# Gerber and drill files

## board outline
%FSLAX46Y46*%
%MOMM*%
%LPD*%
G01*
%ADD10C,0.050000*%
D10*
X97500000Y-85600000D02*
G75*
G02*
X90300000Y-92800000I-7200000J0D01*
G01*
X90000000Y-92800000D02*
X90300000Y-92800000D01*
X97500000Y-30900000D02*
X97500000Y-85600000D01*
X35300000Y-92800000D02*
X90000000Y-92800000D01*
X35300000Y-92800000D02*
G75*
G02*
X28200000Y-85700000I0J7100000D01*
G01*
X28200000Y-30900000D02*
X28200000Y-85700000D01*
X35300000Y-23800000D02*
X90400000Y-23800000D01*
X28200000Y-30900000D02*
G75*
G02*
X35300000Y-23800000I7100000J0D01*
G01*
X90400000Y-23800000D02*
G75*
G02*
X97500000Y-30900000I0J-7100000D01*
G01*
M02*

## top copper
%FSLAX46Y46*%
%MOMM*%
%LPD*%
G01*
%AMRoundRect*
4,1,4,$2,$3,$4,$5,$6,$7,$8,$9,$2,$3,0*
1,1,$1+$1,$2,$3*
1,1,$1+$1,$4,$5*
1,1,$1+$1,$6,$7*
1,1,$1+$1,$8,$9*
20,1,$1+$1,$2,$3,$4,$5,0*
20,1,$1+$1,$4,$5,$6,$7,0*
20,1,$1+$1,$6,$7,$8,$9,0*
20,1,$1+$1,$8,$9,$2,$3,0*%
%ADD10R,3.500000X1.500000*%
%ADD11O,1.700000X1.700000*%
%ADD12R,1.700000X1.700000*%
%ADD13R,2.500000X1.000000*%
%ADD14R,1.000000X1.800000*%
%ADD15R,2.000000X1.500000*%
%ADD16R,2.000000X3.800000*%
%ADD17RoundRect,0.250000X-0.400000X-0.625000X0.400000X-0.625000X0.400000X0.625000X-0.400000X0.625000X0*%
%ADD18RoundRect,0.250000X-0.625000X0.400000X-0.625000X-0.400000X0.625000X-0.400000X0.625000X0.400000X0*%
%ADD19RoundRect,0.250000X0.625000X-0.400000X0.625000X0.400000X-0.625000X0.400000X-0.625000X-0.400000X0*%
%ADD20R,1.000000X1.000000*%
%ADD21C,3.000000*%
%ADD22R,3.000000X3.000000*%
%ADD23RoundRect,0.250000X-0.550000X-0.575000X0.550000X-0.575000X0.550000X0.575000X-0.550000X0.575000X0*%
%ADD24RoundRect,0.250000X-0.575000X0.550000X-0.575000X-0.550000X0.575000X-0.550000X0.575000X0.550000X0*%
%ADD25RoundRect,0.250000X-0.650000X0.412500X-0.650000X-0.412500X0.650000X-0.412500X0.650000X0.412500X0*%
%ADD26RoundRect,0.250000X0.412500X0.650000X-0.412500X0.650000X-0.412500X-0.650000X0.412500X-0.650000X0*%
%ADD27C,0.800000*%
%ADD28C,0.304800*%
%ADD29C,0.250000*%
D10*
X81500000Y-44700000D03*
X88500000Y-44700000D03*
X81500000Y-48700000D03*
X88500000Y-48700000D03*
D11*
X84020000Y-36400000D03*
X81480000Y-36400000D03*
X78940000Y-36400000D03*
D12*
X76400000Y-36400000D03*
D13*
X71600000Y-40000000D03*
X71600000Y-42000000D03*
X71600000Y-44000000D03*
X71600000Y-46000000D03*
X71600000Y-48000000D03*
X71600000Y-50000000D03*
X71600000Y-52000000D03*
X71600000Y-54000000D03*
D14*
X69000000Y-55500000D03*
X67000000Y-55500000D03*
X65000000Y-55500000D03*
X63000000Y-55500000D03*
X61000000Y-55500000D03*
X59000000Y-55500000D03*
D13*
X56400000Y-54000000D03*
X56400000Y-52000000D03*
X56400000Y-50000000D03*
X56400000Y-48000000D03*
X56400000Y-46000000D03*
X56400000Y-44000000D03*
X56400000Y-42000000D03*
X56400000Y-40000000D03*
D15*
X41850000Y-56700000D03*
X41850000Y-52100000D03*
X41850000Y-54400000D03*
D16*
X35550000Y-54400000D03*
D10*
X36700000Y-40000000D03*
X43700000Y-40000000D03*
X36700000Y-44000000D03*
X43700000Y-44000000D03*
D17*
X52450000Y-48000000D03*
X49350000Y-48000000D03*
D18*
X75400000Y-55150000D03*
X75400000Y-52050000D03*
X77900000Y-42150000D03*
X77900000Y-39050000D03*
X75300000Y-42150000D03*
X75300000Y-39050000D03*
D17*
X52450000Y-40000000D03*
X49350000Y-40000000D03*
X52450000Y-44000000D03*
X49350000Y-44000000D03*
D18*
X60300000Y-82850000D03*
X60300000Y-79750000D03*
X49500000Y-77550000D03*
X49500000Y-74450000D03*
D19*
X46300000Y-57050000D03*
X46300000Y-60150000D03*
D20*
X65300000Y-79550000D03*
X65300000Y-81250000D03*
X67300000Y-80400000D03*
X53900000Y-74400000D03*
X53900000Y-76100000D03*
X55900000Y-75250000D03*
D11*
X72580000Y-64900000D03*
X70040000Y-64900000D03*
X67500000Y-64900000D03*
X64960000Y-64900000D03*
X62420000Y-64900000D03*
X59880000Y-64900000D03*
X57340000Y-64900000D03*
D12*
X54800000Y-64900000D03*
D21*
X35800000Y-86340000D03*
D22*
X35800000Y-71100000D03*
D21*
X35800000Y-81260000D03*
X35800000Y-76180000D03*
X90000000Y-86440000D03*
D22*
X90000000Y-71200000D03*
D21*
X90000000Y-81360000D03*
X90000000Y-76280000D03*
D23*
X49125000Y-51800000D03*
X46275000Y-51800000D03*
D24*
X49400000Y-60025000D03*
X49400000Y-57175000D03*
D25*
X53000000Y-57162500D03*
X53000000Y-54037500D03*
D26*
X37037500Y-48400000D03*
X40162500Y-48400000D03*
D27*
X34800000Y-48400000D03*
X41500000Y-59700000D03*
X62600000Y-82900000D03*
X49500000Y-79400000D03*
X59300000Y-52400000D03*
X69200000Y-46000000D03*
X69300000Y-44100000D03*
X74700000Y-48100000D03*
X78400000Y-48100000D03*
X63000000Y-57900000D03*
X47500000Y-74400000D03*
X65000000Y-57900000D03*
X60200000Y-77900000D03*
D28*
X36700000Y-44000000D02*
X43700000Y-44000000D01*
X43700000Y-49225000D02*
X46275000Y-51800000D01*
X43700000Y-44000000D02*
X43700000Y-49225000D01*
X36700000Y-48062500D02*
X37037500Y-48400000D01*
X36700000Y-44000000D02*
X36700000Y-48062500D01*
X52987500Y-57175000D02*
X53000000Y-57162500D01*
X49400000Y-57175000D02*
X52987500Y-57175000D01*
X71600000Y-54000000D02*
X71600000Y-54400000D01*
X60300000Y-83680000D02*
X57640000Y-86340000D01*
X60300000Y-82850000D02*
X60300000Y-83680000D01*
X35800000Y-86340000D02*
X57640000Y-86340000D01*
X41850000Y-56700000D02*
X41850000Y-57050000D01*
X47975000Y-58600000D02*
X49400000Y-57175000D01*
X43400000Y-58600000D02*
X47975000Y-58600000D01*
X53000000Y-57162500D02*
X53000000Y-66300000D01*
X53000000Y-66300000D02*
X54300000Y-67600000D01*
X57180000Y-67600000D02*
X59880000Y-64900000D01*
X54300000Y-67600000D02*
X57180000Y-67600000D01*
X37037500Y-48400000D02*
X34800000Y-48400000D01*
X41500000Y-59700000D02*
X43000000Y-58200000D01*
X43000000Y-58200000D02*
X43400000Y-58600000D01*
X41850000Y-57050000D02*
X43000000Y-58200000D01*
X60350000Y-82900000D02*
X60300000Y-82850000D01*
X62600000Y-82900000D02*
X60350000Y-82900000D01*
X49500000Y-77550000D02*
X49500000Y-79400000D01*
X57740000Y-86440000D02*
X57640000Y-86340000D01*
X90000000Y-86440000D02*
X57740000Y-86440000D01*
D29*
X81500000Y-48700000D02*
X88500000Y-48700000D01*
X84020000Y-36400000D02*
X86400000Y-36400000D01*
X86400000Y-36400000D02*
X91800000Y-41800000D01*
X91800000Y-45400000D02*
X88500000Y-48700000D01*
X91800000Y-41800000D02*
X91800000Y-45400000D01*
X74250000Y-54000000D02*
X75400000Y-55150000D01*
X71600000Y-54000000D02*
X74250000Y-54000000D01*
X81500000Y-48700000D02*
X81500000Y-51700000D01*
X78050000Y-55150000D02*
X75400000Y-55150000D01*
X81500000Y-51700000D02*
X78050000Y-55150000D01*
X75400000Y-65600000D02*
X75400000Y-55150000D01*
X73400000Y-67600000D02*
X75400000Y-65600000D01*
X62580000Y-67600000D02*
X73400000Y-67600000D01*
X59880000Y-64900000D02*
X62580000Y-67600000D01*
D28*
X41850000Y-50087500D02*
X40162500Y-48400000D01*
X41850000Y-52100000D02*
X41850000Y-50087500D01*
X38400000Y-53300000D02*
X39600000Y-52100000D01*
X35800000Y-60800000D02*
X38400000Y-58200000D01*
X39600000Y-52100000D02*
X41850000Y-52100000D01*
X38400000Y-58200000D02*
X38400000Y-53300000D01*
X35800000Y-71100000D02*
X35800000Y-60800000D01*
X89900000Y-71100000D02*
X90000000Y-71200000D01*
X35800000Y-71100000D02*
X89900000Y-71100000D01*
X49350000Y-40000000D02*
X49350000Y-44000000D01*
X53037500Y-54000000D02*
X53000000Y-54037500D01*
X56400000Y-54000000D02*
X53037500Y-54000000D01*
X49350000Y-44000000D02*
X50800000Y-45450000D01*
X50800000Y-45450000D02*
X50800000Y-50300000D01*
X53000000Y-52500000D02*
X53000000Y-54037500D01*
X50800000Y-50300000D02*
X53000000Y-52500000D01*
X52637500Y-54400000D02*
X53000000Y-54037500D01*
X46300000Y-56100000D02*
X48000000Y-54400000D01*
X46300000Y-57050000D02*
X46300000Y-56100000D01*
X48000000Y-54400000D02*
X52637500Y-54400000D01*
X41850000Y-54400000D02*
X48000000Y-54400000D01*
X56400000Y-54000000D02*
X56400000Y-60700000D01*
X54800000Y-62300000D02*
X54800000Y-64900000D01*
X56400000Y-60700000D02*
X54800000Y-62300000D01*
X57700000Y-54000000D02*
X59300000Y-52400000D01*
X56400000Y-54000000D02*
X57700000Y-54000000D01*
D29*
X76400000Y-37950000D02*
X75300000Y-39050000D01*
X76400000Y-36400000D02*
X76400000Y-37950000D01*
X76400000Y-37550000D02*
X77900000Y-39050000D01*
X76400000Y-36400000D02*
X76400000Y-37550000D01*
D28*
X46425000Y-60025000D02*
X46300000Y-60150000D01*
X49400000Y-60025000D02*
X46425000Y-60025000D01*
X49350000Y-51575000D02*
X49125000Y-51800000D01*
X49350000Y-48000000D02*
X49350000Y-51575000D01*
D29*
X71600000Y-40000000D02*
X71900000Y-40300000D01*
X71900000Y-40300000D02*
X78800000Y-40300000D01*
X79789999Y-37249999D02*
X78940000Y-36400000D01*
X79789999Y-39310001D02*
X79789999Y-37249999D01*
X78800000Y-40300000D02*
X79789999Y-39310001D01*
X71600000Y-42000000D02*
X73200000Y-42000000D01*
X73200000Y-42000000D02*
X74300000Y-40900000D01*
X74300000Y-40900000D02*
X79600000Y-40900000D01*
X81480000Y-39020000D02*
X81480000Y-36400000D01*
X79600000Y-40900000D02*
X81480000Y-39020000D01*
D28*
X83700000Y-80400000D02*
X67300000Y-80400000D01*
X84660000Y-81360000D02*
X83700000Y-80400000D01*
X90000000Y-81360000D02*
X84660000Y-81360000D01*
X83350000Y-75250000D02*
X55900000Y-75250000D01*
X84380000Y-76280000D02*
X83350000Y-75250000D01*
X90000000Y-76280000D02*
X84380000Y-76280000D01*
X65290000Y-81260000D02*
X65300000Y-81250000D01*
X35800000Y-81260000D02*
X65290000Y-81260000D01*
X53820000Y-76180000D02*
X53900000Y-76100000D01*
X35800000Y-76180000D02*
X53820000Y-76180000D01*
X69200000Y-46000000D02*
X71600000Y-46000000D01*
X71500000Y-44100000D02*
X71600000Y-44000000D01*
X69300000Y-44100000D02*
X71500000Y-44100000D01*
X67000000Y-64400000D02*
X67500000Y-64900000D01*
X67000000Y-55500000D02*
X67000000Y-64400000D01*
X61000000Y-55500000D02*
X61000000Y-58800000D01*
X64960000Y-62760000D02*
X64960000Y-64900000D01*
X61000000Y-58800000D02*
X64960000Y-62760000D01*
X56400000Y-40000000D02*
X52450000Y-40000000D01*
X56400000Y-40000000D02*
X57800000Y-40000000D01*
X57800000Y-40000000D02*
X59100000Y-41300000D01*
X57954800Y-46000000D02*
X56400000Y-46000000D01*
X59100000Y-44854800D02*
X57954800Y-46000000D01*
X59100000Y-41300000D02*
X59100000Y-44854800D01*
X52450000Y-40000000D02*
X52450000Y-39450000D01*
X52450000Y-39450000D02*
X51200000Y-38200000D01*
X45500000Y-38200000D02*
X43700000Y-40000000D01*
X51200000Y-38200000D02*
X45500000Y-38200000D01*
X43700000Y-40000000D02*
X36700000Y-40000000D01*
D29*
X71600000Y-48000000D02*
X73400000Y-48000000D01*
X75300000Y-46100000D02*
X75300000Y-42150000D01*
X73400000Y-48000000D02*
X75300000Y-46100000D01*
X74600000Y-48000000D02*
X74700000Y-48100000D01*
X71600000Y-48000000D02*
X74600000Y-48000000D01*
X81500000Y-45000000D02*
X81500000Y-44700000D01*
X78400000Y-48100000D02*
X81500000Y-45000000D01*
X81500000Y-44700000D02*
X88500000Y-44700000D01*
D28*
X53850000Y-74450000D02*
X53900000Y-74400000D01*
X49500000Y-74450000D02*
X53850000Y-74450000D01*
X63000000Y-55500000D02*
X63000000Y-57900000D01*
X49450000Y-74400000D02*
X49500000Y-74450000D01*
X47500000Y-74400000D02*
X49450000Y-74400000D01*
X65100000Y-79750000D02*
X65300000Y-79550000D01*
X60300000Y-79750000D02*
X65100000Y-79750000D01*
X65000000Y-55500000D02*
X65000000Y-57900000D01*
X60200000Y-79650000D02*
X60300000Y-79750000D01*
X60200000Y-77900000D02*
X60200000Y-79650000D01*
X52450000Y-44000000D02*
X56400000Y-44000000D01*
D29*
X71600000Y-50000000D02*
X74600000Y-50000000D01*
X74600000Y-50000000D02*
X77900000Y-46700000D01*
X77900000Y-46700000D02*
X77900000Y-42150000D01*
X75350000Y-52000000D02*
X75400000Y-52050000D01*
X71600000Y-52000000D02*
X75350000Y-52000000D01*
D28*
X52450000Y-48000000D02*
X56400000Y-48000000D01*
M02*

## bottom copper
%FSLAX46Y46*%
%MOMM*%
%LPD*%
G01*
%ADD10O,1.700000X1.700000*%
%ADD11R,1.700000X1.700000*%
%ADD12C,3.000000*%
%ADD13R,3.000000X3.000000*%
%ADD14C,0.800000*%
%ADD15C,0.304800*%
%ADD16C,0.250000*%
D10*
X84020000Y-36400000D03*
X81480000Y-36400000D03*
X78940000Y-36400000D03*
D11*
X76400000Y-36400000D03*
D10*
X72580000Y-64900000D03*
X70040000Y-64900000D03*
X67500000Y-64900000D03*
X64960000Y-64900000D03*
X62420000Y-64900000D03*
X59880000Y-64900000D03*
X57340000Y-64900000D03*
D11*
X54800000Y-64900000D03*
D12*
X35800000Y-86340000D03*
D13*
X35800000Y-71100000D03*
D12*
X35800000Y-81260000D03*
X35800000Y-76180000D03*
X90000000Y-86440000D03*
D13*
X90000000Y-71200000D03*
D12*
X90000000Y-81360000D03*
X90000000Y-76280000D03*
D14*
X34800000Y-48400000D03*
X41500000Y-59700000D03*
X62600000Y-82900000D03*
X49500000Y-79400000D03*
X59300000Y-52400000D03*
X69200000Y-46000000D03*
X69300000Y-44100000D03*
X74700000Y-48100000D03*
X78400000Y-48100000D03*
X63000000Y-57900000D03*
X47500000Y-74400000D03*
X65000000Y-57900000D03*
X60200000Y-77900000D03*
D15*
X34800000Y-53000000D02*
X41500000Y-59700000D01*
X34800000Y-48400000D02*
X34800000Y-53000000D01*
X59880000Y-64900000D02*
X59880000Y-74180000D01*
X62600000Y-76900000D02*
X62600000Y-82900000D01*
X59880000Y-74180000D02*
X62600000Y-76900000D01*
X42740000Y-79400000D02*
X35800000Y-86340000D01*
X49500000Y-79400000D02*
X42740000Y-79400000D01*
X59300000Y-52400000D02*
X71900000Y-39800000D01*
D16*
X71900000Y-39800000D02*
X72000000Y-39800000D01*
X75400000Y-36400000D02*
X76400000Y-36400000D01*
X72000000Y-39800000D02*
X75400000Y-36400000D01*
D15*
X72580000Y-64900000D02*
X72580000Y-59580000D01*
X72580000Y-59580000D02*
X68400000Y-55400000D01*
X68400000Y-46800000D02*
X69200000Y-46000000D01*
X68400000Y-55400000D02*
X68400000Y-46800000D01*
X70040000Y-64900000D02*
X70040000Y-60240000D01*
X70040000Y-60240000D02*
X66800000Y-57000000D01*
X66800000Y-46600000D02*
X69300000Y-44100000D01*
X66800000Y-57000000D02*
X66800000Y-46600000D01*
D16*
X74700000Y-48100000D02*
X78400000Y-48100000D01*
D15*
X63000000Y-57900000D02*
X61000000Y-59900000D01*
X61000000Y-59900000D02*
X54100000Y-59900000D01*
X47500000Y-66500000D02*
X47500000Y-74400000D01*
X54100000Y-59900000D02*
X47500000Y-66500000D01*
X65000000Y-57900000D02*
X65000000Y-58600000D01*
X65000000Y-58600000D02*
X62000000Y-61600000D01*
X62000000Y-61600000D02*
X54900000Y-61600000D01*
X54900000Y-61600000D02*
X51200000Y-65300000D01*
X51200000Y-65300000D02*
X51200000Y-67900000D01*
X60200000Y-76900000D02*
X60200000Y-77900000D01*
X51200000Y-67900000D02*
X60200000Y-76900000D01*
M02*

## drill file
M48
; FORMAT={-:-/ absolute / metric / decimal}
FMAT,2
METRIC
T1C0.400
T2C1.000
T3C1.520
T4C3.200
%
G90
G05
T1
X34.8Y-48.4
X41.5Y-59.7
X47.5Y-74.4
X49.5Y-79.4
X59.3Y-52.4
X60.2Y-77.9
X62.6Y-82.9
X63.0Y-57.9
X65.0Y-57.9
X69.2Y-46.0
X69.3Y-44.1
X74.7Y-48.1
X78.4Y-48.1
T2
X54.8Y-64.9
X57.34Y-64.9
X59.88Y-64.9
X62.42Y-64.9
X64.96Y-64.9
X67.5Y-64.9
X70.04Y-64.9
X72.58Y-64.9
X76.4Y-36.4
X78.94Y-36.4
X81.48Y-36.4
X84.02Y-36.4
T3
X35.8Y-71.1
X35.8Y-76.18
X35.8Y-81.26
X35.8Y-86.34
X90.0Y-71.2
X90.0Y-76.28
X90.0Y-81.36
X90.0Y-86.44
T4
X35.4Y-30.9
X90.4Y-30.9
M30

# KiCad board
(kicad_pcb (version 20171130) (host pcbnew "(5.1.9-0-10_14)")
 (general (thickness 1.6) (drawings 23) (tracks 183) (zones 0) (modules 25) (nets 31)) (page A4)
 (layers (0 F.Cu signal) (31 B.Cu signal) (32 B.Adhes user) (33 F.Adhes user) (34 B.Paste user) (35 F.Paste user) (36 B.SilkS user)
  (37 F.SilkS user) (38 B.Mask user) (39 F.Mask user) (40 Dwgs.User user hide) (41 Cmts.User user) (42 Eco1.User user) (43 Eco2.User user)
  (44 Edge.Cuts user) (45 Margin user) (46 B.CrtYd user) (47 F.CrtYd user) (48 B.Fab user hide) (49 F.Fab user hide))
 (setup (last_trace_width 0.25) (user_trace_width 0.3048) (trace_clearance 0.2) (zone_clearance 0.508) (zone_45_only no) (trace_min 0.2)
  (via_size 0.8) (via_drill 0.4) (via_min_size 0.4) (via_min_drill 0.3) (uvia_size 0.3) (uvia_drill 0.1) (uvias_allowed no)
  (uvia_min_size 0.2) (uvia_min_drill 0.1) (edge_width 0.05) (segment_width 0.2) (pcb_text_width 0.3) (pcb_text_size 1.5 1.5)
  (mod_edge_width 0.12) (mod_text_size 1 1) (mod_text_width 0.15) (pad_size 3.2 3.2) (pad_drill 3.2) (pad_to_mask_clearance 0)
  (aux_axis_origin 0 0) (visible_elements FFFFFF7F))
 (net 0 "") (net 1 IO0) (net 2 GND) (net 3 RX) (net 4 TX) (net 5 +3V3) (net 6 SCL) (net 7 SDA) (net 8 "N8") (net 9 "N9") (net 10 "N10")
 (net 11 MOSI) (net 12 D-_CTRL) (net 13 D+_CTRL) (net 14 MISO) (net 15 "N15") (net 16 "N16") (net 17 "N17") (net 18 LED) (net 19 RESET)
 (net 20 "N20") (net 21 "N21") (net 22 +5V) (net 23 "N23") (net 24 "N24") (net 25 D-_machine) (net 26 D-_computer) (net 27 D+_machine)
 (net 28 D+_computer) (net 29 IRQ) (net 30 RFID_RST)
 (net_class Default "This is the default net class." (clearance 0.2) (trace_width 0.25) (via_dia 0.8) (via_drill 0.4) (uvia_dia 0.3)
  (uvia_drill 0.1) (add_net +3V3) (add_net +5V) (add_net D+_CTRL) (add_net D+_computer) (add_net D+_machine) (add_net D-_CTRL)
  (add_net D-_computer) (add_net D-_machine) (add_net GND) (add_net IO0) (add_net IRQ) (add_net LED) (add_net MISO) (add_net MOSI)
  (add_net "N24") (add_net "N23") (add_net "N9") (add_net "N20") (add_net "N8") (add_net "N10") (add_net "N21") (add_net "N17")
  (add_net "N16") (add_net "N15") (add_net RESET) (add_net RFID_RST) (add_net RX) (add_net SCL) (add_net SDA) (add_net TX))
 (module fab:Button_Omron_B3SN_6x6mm (layer F.Cu) (at 85 46.7)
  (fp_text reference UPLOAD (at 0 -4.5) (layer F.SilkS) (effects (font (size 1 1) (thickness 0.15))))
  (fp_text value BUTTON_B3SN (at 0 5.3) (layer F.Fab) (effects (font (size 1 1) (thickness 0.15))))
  (pad 1 smd rect (at -3.5 -2) (size 3.5 1.5) (layers F.Cu F.Paste F.Mask) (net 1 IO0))
  (pad 1 smd rect (at 3.5 -2) (size 3.5 1.5) (layers F.Cu F.Paste F.Mask) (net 1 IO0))
  (pad 2 smd rect (at -3.5 2) (size 3.5 1.5) (layers F.Cu F.Paste F.Mask) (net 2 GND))
  (pad 2 smd rect (at 3.5 2) (size 3.5 1.5) (layers F.Cu F.Paste F.Mask) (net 2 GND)))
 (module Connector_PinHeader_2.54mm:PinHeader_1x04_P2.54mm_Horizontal (layer F.Cu) (at 76.4 36.4 90)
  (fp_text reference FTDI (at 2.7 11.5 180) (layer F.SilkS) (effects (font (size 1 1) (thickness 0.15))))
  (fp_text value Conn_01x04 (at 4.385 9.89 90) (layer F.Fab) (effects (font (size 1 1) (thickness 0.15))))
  (pad 4 thru_hole oval (at 0 7.62 90) (size 1.7 1.7) (drill 1) (layers *.Cu *.Mask) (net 2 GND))
  (pad 3 thru_hole oval (at 0 5.08 90) (size 1.7 1.7) (drill 1) (layers *.Cu *.Mask) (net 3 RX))
  (pad 2 thru_hole oval (at 0 2.54 90) (size 1.7 1.7) (drill 1) (layers *.Cu *.Mask) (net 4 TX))
  (pad 1 thru_hole rect (at 0 0 90) (size 1.7 1.7) (drill 1) (layers *.Cu *.Mask) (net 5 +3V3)))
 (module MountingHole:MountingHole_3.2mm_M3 (layer F.Cu) (at 90.4 30.9)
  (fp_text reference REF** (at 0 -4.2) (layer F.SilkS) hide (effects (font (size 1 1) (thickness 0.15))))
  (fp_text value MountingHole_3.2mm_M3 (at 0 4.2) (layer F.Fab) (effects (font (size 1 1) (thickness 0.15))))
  (pad 1 np_thru_hole circle (at 0 0) (size 3.2 3.2) (drill 3.2) (layers *.Cu *.Mask)))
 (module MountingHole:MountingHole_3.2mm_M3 (layer F.Cu) (at 35.4 30.9)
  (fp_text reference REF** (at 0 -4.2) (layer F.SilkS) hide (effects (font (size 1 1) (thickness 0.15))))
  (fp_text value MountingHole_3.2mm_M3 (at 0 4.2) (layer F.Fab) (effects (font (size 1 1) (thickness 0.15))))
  (pad 1 np_thru_hole circle (at 0 0) (size 3.2 3.2) (drill 3.2) (layers *.Cu *.Mask)))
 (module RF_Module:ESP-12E (layer F.Cu) (at 64 43.5)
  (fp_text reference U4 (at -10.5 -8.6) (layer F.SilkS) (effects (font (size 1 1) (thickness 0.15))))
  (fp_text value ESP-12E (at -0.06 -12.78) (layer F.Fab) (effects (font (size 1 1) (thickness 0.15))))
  (pad 22 smd rect (at 7.6 -3.5) (size 2.5 1) (layers F.Cu F.Paste F.Mask) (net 4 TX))
  (pad 21 smd rect (at 7.6 -1.5) (size 2.5 1) (layers F.Cu F.Paste F.Mask) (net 3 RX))
  (pad 20 smd rect (at 7.6 0.5) (size 2.5 1) (layers F.Cu F.Paste F.Mask) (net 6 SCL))
  (pad 19 smd rect (at 7.6 2.5) (size 2.5 1) (layers F.Cu F.Paste F.Mask) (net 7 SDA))
  (pad 18 smd rect (at 7.6 4.5) (size 2.5 1) (layers F.Cu F.Paste F.Mask) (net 1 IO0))
  (pad 17 smd rect (at 7.6 6.5) (size 2.5 1) (layers F.Cu F.Paste F.Mask) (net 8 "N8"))
  (pad 16 smd rect (at 7.6 8.5) (size 2.5 1) (layers F.Cu F.Paste F.Mask) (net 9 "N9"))
  (pad 15 smd rect (at 7.6 10.5) (size 2.5 1) (layers F.Cu F.Paste F.Mask) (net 2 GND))
  (pad 14 smd rect (at 5 12) (size 1 1.8) (layers F.Cu F.Paste F.Mask) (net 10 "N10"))
  (pad 13 smd rect (at 3 12) (size 1 1.8) (layers F.Cu F.Paste F.Mask) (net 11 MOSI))
  (pad 12 smd rect (at 1 12) (size 1 1.8) (layers F.Cu F.Paste F.Mask) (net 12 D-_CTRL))
  (pad 11 smd rect (at -1 12) (size 1 1.8) (layers F.Cu F.Paste F.Mask) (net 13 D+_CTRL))
  (pad 10 smd rect (at -3 12) (size 1 1.8) (layers F.Cu F.Paste F.Mask) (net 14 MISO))
  (pad 9 smd rect (at -5 12) (size 1 1.8) (layers F.Cu F.Paste F.Mask) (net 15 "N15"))
  (pad 8 smd rect (at -7.6 10.5) (size 2.5 1) (layers F.Cu F.Paste F.Mask) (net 5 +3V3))
  (pad 7 smd rect (at -7.6 8.5) (size 2.5 1) (layers F.Cu F.Paste F.Mask) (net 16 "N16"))
  (pad 6 smd rect (at -7.6 6.5) (size 2.5 1) (layers F.Cu F.Paste F.Mask) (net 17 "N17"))
  (pad 5 smd rect (at -7.6 4.5) (size 2.5 1) (layers F.Cu F.Paste F.Mask) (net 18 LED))
  (pad 4 smd rect (at -7.6 2.5) (size 2.5 1) (layers F.Cu F.Paste F.Mask) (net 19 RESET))
  (pad 3 smd rect (at -7.6 0.5) (size 2.5 1) (layers F.Cu F.Paste F.Mask) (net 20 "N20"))
  (pad 2 smd rect (at -7.6 -1.5) (size 2.5 1) (layers F.Cu F.Paste F.Mask) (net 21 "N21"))
  (pad 1 smd rect (at -7.6 -3.5) (size 2.5 1) (layers F.Cu F.Paste F.Mask) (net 19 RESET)))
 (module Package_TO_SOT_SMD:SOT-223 (layer F.Cu) (at 38.7 54.4 180)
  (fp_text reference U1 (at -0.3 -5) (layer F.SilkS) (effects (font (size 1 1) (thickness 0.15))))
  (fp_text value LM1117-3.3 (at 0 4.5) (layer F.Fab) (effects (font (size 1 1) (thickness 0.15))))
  (pad 1 smd rect (at -3.15 -2.3 180) (size 2 1.5) (layers F.Cu F.Paste F.Mask) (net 2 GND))
  (pad 3 smd rect (at -3.15 2.3 180) (size 2 1.5) (layers F.Cu F.Paste F.Mask) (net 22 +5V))
  (pad 2 smd rect (at -3.15 0 180) (size 2 1.5) (layers F.Cu F.Paste F.Mask) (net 5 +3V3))
  (pad 4 smd rect (at 3.15 0 180) (size 2 3.8) (layers F.Cu F.Paste F.Mask)))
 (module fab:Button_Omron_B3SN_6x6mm (layer F.Cu) (at 40.2 42)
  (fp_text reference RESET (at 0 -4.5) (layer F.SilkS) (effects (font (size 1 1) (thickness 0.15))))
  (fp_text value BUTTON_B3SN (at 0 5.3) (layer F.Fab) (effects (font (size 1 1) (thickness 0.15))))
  (pad 1 smd rect (at -3.5 -2) (size 3.5 1.5) (layers F.Cu F.Paste F.Mask) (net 19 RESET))
  (pad 1 smd rect (at 3.5 -2) (size 3.5 1.5) (layers F.Cu F.Paste F.Mask) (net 19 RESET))
  (pad 2 smd rect (at -3.5 2) (size 3.5 1.5) (layers F.Cu F.Paste F.Mask) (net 2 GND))
  (pad 2 smd rect (at 3.5 2) (size 3.5 1.5) (layers F.Cu F.Paste F.Mask) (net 2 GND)))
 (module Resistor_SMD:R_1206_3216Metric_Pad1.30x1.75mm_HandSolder (layer F.Cu) (at 50.9 48)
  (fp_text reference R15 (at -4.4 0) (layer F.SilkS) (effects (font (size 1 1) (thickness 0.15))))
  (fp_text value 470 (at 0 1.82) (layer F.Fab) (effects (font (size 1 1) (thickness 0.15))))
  (pad 2 smd roundrect (at 1.55 0) (size 1.3 1.75) (layers F.Cu F.Paste F.Mask) (roundrect_rratio 0.192308) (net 18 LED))
  (pad 1 smd roundrect (at -1.55 0) (size 1.3 1.75) (layers F.Cu F.Paste F.Mask) (roundrect_rratio 0.192308) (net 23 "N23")))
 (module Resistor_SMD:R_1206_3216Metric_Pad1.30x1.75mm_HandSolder (layer F.Cu) (at 75.4 53.6 270)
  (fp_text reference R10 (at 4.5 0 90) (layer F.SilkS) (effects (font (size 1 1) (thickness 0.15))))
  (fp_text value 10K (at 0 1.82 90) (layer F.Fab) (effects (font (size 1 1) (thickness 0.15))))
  (pad 2 smd roundrect (at 1.55 0 270) (size 1.3 1.75) (layers F.Cu F.Paste F.Mask) (roundrect_rratio 0.192308) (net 2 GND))
  (pad 1 smd roundrect (at -1.55 0 270) (size 1.3 1.75) (layers F.Cu F.Paste F.Mask) (roundrect_rratio 0.192308) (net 9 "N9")))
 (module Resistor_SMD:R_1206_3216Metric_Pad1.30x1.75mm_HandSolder (layer F.Cu) (at 77.9 40.6 270)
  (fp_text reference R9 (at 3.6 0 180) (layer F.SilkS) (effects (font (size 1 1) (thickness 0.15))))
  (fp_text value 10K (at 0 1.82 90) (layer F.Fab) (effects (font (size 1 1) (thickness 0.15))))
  (pad 2 smd roundrect (at 1.55 0 270) (size 1.3 1.75) (layers F.Cu F.Paste F.Mask) (roundrect_rratio 0.192308) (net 8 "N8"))
  (pad 1 smd roundrect (at -1.55 0 270) (size 1.3 1.75) (layers F.Cu F.Paste F.Mask) (roundrect_rratio 0.192308) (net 5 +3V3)))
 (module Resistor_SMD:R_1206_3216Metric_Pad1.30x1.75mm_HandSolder (layer F.Cu) (at 75.3 40.6 270)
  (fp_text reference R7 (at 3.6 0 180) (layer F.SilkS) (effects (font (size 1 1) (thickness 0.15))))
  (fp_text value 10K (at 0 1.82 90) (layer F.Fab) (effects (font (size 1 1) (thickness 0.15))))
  (pad 2 smd roundrect (at 1.55 0 270) (size 1.3 1.75) (layers F.Cu F.Paste F.Mask) (roundrect_rratio 0.192308) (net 1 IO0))
  (pad 1 smd roundrect (at -1.55 0 270) (size 1.3 1.75) (layers F.Cu F.Paste F.Mask) (roundrect_rratio 0.192308) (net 5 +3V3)))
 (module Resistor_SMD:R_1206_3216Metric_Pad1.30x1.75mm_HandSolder (layer F.Cu) (at 50.9 40)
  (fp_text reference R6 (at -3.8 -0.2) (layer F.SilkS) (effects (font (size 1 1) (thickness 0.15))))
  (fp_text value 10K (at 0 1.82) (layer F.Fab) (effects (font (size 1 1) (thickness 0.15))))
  (pad 2 smd roundrect (at 1.55 0) (size 1.3 1.75) (layers F.Cu F.Paste F.Mask) (roundrect_rratio 0.192308) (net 19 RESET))
  (pad 1 smd roundrect (at -1.55 0) (size 1.3 1.75) (layers F.Cu F.Paste F.Mask) (roundrect_rratio 0.192308) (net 5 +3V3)))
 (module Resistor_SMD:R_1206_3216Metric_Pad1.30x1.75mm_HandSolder (layer F.Cu) (at 50.9 44)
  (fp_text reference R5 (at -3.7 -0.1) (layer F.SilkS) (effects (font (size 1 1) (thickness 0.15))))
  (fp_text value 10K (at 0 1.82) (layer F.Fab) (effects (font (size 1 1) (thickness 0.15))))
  (pad 2 smd roundrect (at 1.55 0) (size 1.3 1.75) (layers F.Cu F.Paste F.Mask) (roundrect_rratio 0.192308) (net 20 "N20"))
  (pad 1 smd roundrect (at -1.55 0) (size 1.3 1.75) (layers F.Cu F.Paste F.Mask) (roundrect_rratio 0.192308) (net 5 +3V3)))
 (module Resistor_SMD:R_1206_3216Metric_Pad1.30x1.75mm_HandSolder (layer F.Cu) (at 60.3 81.3 270)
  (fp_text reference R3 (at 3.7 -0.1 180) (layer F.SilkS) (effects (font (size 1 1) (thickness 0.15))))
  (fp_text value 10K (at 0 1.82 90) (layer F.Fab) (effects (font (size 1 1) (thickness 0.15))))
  (pad 2 smd roundrect (at 1.55 0 270) (size 1.3 1.75) (layers F.Cu F.Paste F.Mask) (roundrect_rratio 0.192308) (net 2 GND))
  (pad 1 smd roundrect (at -1.55 0 270) (size 1.3 1.75) (layers F.Cu F.Paste F.Mask) (roundrect_rratio 0.192308) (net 12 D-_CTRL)))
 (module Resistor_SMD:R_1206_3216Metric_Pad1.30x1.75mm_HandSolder (layer F.Cu) (at 49.5 76 270)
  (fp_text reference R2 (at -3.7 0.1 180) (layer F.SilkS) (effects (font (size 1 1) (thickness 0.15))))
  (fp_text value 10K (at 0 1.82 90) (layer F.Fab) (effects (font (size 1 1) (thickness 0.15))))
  (pad 2 smd roundrect (at 1.55 0 270) (size 1.3 1.75) (layers F.Cu F.Paste F.Mask) (roundrect_rratio 0.192308) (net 2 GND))
  (pad 1 smd roundrect (at -1.55 0 270) (size 1.3 1.75) (layers F.Cu F.Paste F.Mask) (roundrect_rratio 0.192308) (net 13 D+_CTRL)))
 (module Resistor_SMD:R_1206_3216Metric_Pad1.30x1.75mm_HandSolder (layer F.Cu) (at 46.3 58.6 90)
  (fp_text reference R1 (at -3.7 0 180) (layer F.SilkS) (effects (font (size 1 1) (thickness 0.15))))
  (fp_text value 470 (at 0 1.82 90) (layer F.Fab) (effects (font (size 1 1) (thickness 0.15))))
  (pad 2 smd roundrect (at 1.55 0 90) (size 1.3 1.75) (layers F.Cu F.Paste F.Mask) (roundrect_rratio 0.192308) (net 5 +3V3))
  (pad 1 smd roundrect (at -1.55 0 90) (size 1.3 1.75) (layers F.Cu F.Paste F.Mask) (roundrect_rratio 0.192308) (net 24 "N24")))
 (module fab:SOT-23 (layer F.Cu) (at 66.3 80.4)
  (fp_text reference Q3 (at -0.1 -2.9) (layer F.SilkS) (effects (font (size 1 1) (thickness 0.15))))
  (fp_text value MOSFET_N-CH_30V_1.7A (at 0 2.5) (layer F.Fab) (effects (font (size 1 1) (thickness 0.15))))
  (pad 1 smd rect (at -1 -0.85) (size 1 1) (layers F.Cu F.Paste F.Mask) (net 12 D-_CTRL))
  (pad 2 smd rect (at -1 0.85) (size 1 1) (layers F.Cu F.Paste F.Mask) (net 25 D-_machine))
  (pad 3 smd rect (at 1 0) (size 1 1) (layers F.Cu F.Paste F.Mask) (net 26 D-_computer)))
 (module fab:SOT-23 (layer F.Cu) (at 54.9 75.25)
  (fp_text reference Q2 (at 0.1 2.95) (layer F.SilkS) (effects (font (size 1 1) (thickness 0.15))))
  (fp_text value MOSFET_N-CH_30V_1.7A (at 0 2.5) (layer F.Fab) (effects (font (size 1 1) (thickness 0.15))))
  (pad 1 smd rect (at -1 -0.85) (size 1 1) (layers F.Cu F.Paste F.Mask) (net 13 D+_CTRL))
  (pad 2 smd rect (at -1 0.85) (size 1 1) (layers F.Cu F.Paste F.Mask) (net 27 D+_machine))
  (pad 3 smd rect (at 1 0) (size 1 1) (layers F.Cu F.Paste F.Mask) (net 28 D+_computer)))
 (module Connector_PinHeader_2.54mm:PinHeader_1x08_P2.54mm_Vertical (layer F.Cu) (at 54.8 64.9 90)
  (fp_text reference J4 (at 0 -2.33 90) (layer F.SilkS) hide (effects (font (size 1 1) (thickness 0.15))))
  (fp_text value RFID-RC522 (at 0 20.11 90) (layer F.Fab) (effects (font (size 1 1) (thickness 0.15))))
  (pad 8 thru_hole oval (at 0 17.78 90) (size 1.7 1.7) (drill 1) (layers *.Cu *.Mask) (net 7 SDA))
  (pad 7 thru_hole oval (at 0 15.24 90) (size 1.7 1.7) (drill 1) (layers *.Cu *.Mask) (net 6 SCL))
  (pad 6 thru_hole oval (at 0 12.7 90) (size 1.7 1.7) (drill 1) (layers *.Cu *.Mask) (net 11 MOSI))
  (pad 5 thru_hole oval (at 0 10.16 90) (size 1.7 1.7) (drill 1) (layers *.Cu *.Mask) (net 14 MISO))
  (pad 4 thru_hole oval (at 0 7.62 90) (size 1.7 1.7) (drill 1) (layers *.Cu *.Mask) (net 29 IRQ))
  (pad 3 thru_hole oval (at 0 5.08 90) (size 1.7 1.7) (drill 1) (layers *.Cu *.Mask) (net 2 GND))
  (pad 2 thru_hole oval (at 0 2.54 90) (size 1.7 1.7) (drill 1) (layers *.Cu *.Mask) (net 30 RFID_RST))
  (pad 1 thru_hole rect (at 0 0 90) (size 1.7 1.7) (drill 1) (layers *.Cu *.Mask) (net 5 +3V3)))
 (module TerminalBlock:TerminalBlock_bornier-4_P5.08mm (layer F.Cu) (at 35.8 71.1 270)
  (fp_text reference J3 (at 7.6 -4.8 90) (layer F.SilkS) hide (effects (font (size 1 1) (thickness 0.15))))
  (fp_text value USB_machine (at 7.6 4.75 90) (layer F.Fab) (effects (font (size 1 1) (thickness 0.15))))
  (pad 4 thru_hole circle (at 15.24 0 270) (size 3 3) (drill 1.52) (layers *.Cu *.Mask) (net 2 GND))
  (pad 1 thru_hole rect (at 0 0 270) (size 3 3) (drill 1.52) (layers *.Cu *.Mask) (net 22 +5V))
  (pad 3 thru_hole circle (at 10.16 0 270) (size 3 3) (drill 1.52) (layers *.Cu *.Mask) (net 25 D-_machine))
  (pad 2 thru_hole circle (at 5.08 0 270) (size 3 3) (drill 1.52) (layers *.Cu *.Mask) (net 27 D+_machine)))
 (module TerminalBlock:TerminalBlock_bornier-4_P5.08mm (layer F.Cu) (at 90 71.2 270)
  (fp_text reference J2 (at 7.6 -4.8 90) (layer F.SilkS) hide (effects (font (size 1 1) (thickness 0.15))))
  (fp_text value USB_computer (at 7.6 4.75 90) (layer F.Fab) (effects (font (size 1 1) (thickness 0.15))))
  (pad 4 thru_hole circle (at 15.24 0 270) (size 3 3) (drill 1.52) (layers *.Cu *.Mask) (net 2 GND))
  (pad 1 thru_hole rect (at 0 0 270) (size 3 3) (drill 1.52) (layers *.Cu *.Mask) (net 22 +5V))
  (pad 3 thru_hole circle (at 10.16 0 270) (size 3 3) (drill 1.52) (layers *.Cu *.Mask) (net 26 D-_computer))
  (pad 2 thru_hole circle (at 5.08 0 270) (size 3 3) (drill 1.52) (layers *.Cu *.Mask) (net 28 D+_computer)))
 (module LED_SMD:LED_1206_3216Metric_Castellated (layer F.Cu) (at 47.7 51.8)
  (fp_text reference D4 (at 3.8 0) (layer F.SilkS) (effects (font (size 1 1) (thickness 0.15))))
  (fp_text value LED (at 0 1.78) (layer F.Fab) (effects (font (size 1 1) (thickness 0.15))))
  (pad 2 smd roundrect (at 1.425 0) (size 1.6 1.65) (layers F.Cu F.Paste F.Mask) (roundrect_rratio 0.15625) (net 23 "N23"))
  (pad 1 smd roundrect (at -1.425 0) (size 1.6 1.65) (layers F.Cu F.Paste F.Mask) (roundrect_rratio 0.15625) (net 2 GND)))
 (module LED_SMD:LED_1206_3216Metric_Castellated (layer F.Cu) (at 49.4 58.6 270)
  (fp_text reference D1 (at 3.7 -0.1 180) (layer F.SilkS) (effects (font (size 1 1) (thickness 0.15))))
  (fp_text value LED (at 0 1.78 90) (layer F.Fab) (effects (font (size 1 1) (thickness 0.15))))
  (pad 2 smd roundrect (at 1.425 0 270) (size 1.6 1.65) (layers F.Cu F.Paste F.Mask) (roundrect_rratio 0.15625) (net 24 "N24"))
  (pad 1 smd roundrect (at -1.425 0 270) (size 1.6 1.65) (layers F.Cu F.Paste F.Mask) (roundrect_rratio 0.15625) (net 2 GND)))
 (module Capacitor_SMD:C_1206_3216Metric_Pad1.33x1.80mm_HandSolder (layer F.Cu) (at 53 55.6 270)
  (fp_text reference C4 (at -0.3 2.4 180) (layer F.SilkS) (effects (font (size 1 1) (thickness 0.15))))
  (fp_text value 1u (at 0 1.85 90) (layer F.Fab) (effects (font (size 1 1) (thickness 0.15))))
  (pad 2 smd roundrect (at 1.5625 0 270) (size 1.325 1.8) (layers F.Cu F.Paste F.Mask) (roundrect_rratio 0.188679) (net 2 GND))
  (pad 1 smd roundrect (at -1.5625 0 270) (size 1.325 1.8) (layers F.Cu F.Paste F.Mask) (roundrect_rratio 0.188679) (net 5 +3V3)))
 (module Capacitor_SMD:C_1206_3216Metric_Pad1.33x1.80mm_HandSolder (layer F.Cu) (at 38.6 48.4 180)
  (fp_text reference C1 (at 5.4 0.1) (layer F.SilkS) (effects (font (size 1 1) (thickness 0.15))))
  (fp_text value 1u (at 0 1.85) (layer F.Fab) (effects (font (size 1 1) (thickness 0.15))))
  (pad 2 smd roundrect (at 1.5625 0 180) (size 1.325 1.8) (layers F.Cu F.Paste F.Mask) (roundrect_rratio 0.188679) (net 2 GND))
  (pad 1 smd roundrect (at -1.5625 0 180) (size 1.325 1.8) (layers F.Cu F.Paste F.Mask) (roundrect_rratio 0.188679) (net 22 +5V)))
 (gr_arc (start 90.3 85.6) (end 90.3 92.8) (angle -90) (layer Edge.Cuts) (width 0.05))
 (gr_line (start 90 92.8) (end 90.3 92.8) (layer Edge.Cuts) (width 0.05))
 (gr_line (start 97.5 30.9) (end 97.5 85.6) (layer Edge.Cuts) (width 0.05))
 (gr_line (start 35.3 92.8) (end 90 92.8) (layer Edge.Cuts) (width 0.05))
 (gr_arc (start 35.3 85.7) (end 28.2 85.7) (angle -90) (layer Edge.Cuts) (width 0.05))
 (gr_line (start 28.2 30.9) (end 28.2 85.7) (layer Edge.Cuts) (width 0.05))
 (gr_line (start 35.3 23.8) (end 90.4 23.8) (layer Edge.Cuts) (width 0.05))
 (gr_arc (start 35.3 30.9) (end 35.3 23.8) (angle -90) (layer Edge.Cuts) (width 0.05))
 (gr_arc (start 90.4 30.9) (end 97.5 30.9) (angle -90) (layer Edge.Cuts) (width 0.05))
 (segment (start 36.7 44) (end 43.7 44) (width 0.3048) (layer F.Cu) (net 2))
 (segment (start 43.7 49.225) (end 46.275 51.8) (width 0.3048) (layer F.Cu) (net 2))
 (segment (start 43.7 44) (end 43.7 49.225) (width 0.3048) (layer F.Cu) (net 2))
 (segment (start 36.7 48.0625) (end 37.0375 48.4) (width 0.3048) (layer F.Cu) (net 2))
 (segment (start 36.7 44) (end 36.7 48.0625) (width 0.3048) (layer F.Cu) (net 2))
 (segment (start 52.9875 57.175) (end 53 57.1625) (width 0.3048) (layer F.Cu) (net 2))
 (segment (start 49.4 57.175) (end 52.9875 57.175) (width 0.3048) (layer F.Cu) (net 2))
 (segment (start 71.6 54) (end 71.6 54.4) (width 0.3048) (layer F.Cu) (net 2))
 (segment (start 60.3 83.68) (end 57.64 86.34) (width 0.3048) (layer F.Cu) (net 2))
 (segment (start 60.3 82.85) (end 60.3 83.68) (width 0.3048) (layer F.Cu) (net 2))
 (segment (start 35.8 86.34) (end 57.64 86.34) (width 0.3048) (layer F.Cu) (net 2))
 (segment (start 41.85 56.7) (end 41.85 57.05) (width 0.3048) (layer F.Cu) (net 2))
 (segment (start 47.975 58.6) (end 49.4 57.175) (width 0.3048) (layer F.Cu) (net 2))
 (segment (start 43.4 58.6) (end 47.975 58.6) (width 0.3048) (layer F.Cu) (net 2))
 (segment (start 53 57.1625) (end 53 66.3) (width 0.3048) (layer F.Cu) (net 2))
 (segment (start 53 66.3) (end 54.3 67.6) (width 0.3048) (layer F.Cu) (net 2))
 (segment (start 57.18 67.6) (end 59.88 64.9) (width 0.3048) (layer F.Cu) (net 2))
 (segment (start 54.3 67.6) (end 57.18 67.6) (width 0.3048) (layer F.Cu) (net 2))
 (via (at 34.8 48.4) (size 0.8) (drill 0.4) (layers F.Cu B.Cu) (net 2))
 (segment (start 37.0375 48.4) (end 34.8 48.4) (width 0.3048) (layer F.Cu) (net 2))
 (segment (start 34.8 53) (end 41.5 59.7) (width 0.3048) (layer B.Cu) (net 2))
 (via (at 41.5 59.7) (size 0.8) (drill 0.4) (layers F.Cu B.Cu) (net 2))
 (segment (start 34.8 48.4) (end 34.8 53) (width 0.3048) (layer B.Cu) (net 2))
 (segment (start 41.5 59.7) (end 43 58.2) (width 0.3048) (layer F.Cu) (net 2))
 (segment (start 43 58.2) (end 43.4 58.6) (width 0.3048) (layer F.Cu) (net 2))
 (segment (start 41.85 57.05) (end 43 58.2) (width 0.3048) (layer F.Cu) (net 2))
 (segment (start 59.88 64.9) (end 59.88 74.18) (width 0.3048) (layer B.Cu) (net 2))
 (via (at 62.6 82.9) (size 0.8) (drill 0.4) (layers F.Cu B.Cu) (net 2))
 (segment (start 62.6 76.9) (end 62.6 82.9) (width 0.3048) (layer B.Cu) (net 2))
 (segment (start 59.88 74.18) (end 62.6 76.9) (width 0.3048) (layer B.Cu) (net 2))
 (segment (start 60.35 82.9) (end 60.3 82.85) (width 0.3048) (layer F.Cu) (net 2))
 (segment (start 62.6 82.9) (end 60.35 82.9) (width 0.3048) (layer F.Cu) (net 2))
 (via (at 49.5 79.4) (size 0.8) (drill 0.4) (layers F.Cu B.Cu) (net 2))
 (segment (start 49.5 77.55) (end 49.5 79.4) (width 0.3048) (layer F.Cu) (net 2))
 (segment (start 42.74 79.4) (end 35.8 86.34) (width 0.3048) (layer B.Cu) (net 2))
 (segment (start 49.5 79.4) (end 42.74 79.4) (width 0.3048) (layer B.Cu) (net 2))
 (segment (start 57.74 86.44) (end 57.64 86.34) (width 0.3048) (layer F.Cu) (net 2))
 (segment (start 90 86.44) (end 57.74 86.44) (width 0.3048) (layer F.Cu) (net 2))
 (segment (start 81.5 48.7) (end 88.5 48.7) (width 0.25) (layer F.Cu) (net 2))
 (segment (start 84.02 36.4) (end 86.4 36.4) (width 0.25) (layer F.Cu) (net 2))
 (segment (start 86.4 36.4) (end 91.8 41.8) (width 0.25) (layer F.Cu) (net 2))
 (segment (start 91.8 45.4) (end 88.5 48.7) (width 0.25) (layer F.Cu) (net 2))
 (segment (start 91.8 41.8) (end 91.8 45.4) (width 0.25) (layer F.Cu) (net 2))
 (segment (start 74.25 54) (end 75.4 55.15) (width 0.25) (layer F.Cu) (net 2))
 (segment (start 71.6 54) (end 74.25 54) (width 0.25) (layer F.Cu) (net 2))
 (segment (start 81.5 48.7) (end 81.5 51.7) (width 0.25) (layer F.Cu) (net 2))
 (segment (start 78.05 55.15) (end 75.4 55.15) (width 0.25) (layer F.Cu) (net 2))
 (segment (start 81.5 51.7) (end 78.05 55.15) (width 0.25) (layer F.Cu) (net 2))
 (segment (start 75.4 65.6) (end 75.4 55.15) (width 0.25) (layer F.Cu) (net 2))
 (segment (start 73.4 67.6) (end 75.4 65.6) (width 0.25) (layer F.Cu) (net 2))
 (segment (start 62.58 67.6) (end 73.4 67.6) (width 0.25) (layer F.Cu) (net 2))
 (segment (start 59.88 64.9) (end 62.58 67.6) (width 0.25) (layer F.Cu) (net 2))
 (segment (start 41.85 50.0875) (end 40.1625 48.4) (width 0.3048) (layer F.Cu) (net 22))
 (segment (start 41.85 52.1) (end 41.85 50.0875) (width 0.3048) (layer F.Cu) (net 22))
 (segment (start 38.4 53.3) (end 39.6 52.1) (width 0.3048) (layer F.Cu) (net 22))
 (segment (start 35.8 60.8) (end 38.4 58.2) (width 0.3048) (layer F.Cu) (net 22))
 (segment (start 39.6 52.1) (end 41.85 52.1) (width 0.3048) (layer F.Cu) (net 22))
 (segment (start 38.4 58.2) (end 38.4 53.3) (width 0.3048) (layer F.Cu) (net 22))
 (segment (start 35.8 71.1) (end 35.8 60.8) (width 0.3048) (layer F.Cu) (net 22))
 (segment (start 89.9 71.1) (end 90 71.2) (width 0.3048) (layer F.Cu) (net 22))
 (segment (start 35.8 71.1) (end 89.9 71.1) (width 0.3048) (layer F.Cu) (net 22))
 (segment (start 49.35 40) (end 49.35 44) (width 0.3048) (layer F.Cu) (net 5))
 (segment (start 53.0375 54) (end 53 54.0375) (width 0.3048) (layer F.Cu) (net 5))
 (segment (start 56.4 54) (end 53.0375 54) (width 0.3048) (layer F.Cu) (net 5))
 (segment (start 49.35 44) (end 50.8 45.45) (width 0.3048) (layer F.Cu) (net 5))
 (segment (start 50.8 45.45) (end 50.8 50.3) (width 0.3048) (layer F.Cu) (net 5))
 (segment (start 53 52.5) (end 53 54.0375) (width 0.3048) (layer F.Cu) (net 5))
 (segment (start 50.8 50.3) (end 53 52.5) (width 0.3048) (layer F.Cu) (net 5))
 (segment (start 52.6375 54.4) (end 53 54.0375) (width 0.3048) (layer F.Cu) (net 5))
 (segment (start 46.3 56.1) (end 48 54.4) (width 0.3048) (layer F.Cu) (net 5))
 (segment (start 46.3 57.05) (end 46.3 56.1) (width 0.3048) (layer F.Cu) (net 5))
 (segment (start 48 54.4) (end 52.6375 54.4) (width 0.3048) (layer F.Cu) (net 5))
 (segment (start 41.85 54.4) (end 48 54.4) (width 0.3048) (layer F.Cu) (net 5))
 (segment (start 56.4 54) (end 56.4 60.7) (width 0.3048) (layer F.Cu) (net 5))
 (segment (start 54.8 62.3) (end 54.8 64.9) (width 0.3048) (layer F.Cu) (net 5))
 (segment (start 56.4 60.7) (end 54.8 62.3) (width 0.3048) (layer F.Cu) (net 5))
 (via (at 59.3 52.4) (size 0.8) (drill 0.4) (layers F.Cu B.Cu) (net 5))
 (segment (start 57.7 54) (end 59.3 52.4) (width 0.3048) (layer F.Cu) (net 5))
 (segment (start 56.4 54) (end 57.7 54) (width 0.3048) (layer F.Cu) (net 5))
 (segment (start 59.3 52.4) (end 71.9 39.8) (width 0.3048) (layer B.Cu) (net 5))
 (segment (start 71.9 39.8) (end 72 39.8) (width 0.25) (layer B.Cu) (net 5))
 (segment (start 75.4 36.4) (end 76.4 36.4) (width 0.25) (layer B.Cu) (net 5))
 (segment (start 72 39.8) (end 75.4 36.4) (width 0.25) (layer B.Cu) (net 5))
 (segment (start 76.4 37.95) (end 75.3 39.05) (width 0.25) (layer F.Cu) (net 5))
 (segment (start 76.4 36.4) (end 76.4 37.95) (width 0.25) (layer F.Cu) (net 5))
 (segment (start 76.4 37.55) (end 77.9 39.05) (width 0.25) (layer F.Cu) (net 5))
 (segment (start 76.4 36.4) (end 76.4 37.55) (width 0.25) (layer F.Cu) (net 5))
 (segment (start 46.425 60.025) (end 46.3 60.15) (width 0.3048) (layer F.Cu) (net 24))
 (segment (start 49.4 60.025) (end 46.425 60.025) (width 0.3048) (layer F.Cu) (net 24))
 (segment (start 49.35 51.575) (end 49.125 51.8) (width 0.3048) (layer F.Cu) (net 23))
 (segment (start 49.35 48) (end 49.35 51.575) (width 0.3048) (layer F.Cu) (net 23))
 (segment (start 71.6 40) (end 71.9 40.3) (width 0.25) (layer F.Cu) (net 4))
 (segment (start 71.9 40.3) (end 78.8 40.3) (width 0.25) (layer F.Cu) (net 4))
 (segment (start 79.789999 37.249999) (end 78.94 36.4) (width 0.25) (layer F.Cu) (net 4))
 (segment (start 79.789999 39.310001) (end 79.789999 37.249999) (width 0.25) (layer F.Cu) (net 4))
 (segment (start 78.8 40.3) (end 79.789999 39.310001) (width 0.25) (layer F.Cu) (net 4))
 (segment (start 71.6 42) (end 73.2 42) (width 0.25) (layer F.Cu) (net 3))
 (segment (start 73.2 42) (end 74.3 40.9) (width 0.25) (layer F.Cu) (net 3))
 (segment (start 74.3 40.9) (end 79.6 40.9) (width 0.25) (layer F.Cu) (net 3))
 (segment (start 81.48 39.02) (end 81.48 36.4) (width 0.25) (layer F.Cu) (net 3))
 (segment (start 79.6 40.9) (end 81.48 39.02) (width 0.25) (layer F.Cu) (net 3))
 (segment (start 83.7 80.4) (end 67.3 80.4) (width 0.3048) (layer F.Cu) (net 26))
 (segment (start 84.66 81.36) (end 83.7 80.4) (width 0.3048) (layer F.Cu) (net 26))
 (segment (start 90 81.36) (end 84.66 81.36) (width 0.3048) (layer F.Cu) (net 26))
 (segment (start 83.35 75.25) (end 55.9 75.25) (width 0.3048) (layer F.Cu) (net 28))
 (segment (start 84.38 76.28) (end 83.35 75.25) (width 0.3048) (layer F.Cu) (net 28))
 (segment (start 90 76.28) (end 84.38 76.28) (width 0.3048) (layer F.Cu) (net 28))
 (segment (start 65.29 81.26) (end 65.3 81.25) (width 0.3048) (layer F.Cu) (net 25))
 (segment (start 35.8 81.26) (end 65.29 81.26) (width 0.3048) (layer F.Cu) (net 25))
 (segment (start 53.82 76.18) (end 53.9 76.1) (width 0.3048) (layer F.Cu) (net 27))
 (segment (start 35.8 76.18) (end 53.82 76.18) (width 0.3048) (layer F.Cu) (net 27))
 (segment (start 72.58 64.9) (end 72.58 59.58) (width 0.3048) (layer B.Cu) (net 7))
 (segment (start 72.58 59.58) (end 68.4 55.4) (width 0.3048) (layer B.Cu) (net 7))
 (via (at 69.2 46) (size 0.8) (drill 0.4) (layers F.Cu B.Cu) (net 7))
 (segment (start 68.4 46.8) (end 69.2 46) (width 0.3048) (layer B.Cu) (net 7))
 (segment (start 68.4 55.4) (end 68.4 46.8) (width 0.3048) (layer B.Cu) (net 7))
 (segment (start 69.2 46) (end 71.6 46) (width 0.3048) (layer F.Cu) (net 7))
 (segment (start 70.04 64.9) (end 70.04 60.24) (width 0.3048) (layer B.Cu) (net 6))
 (segment (start 70.04 60.24) (end 66.8 57) (width 0.3048) (layer B.Cu) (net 6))
 (via (at 69.3 44.1) (size 0.8) (drill 0.4) (layers F.Cu B.Cu) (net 6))
 (segment (start 66.8 46.6) (end 69.3 44.1) (width 0.3048) (layer B.Cu) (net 6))
 (segment (start 66.8 57) (end 66.8 46.6) (width 0.3048) (layer B.Cu) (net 6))
 (segment (start 71.5 44.1) (end 71.6 44) (width 0.3048) (layer F.Cu) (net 6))
 (segment (start 69.3 44.1) (end 71.5 44.1) (width 0.3048) (layer F.Cu) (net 6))
 (segment (start 67 64.4) (end 67.5 64.9) (width 0.3048) (layer F.Cu) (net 11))
 (segment (start 67 55.5) (end 67 64.4) (width 0.3048) (layer F.Cu) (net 11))
 (segment (start 61 55.5) (end 61 58.8) (width 0.3048) (layer F.Cu) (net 14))
 (segment (start 64.96 62.76) (end 64.96 64.9) (width 0.3048) (layer F.Cu) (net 14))
 (segment (start 61 58.8) (end 64.96 62.76) (width 0.3048) (layer F.Cu) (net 14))
 (segment (start 56.4 40) (end 52.45 40) (width 0.3048) (layer F.Cu) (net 19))
 (segment (start 56.4 40) (end 57.8 40) (width 0.3048) (layer F.Cu) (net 19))
 (segment (start 57.8 40) (end 59.1 41.3) (width 0.3048) (layer F.Cu) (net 19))
 (segment (start 57.9548 46) (end 56.4 46) (width 0.3048) (layer F.Cu) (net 19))
 (segment (start 59.1 44.8548) (end 57.9548 46) (width 0.3048) (layer F.Cu) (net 19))
 (segment (start 59.1 41.3) (end 59.1 44.8548) (width 0.3048) (layer F.Cu) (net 19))
 (segment (start 52.45 40) (end 52.45 39.45) (width 0.3048) (layer F.Cu) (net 19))
 (segment (start 52.45 39.45) (end 51.2 38.2) (width 0.3048) (layer F.Cu) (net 19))
 (segment (start 45.5 38.2) (end 43.7 40) (width 0.3048) (layer F.Cu) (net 19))
 (segment (start 51.2 38.2) (end 45.5 38.2) (width 0.3048) (layer F.Cu) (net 19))
 (segment (start 43.7 40) (end 36.7 40) (width 0.3048) (layer F.Cu) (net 19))
 (segment (start 71.6 48) (end 73.4 48) (width 0.25) (layer F.Cu) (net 1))
 (segment (start 75.3 46.1) (end 75.3 42.15) (width 0.25) (layer F.Cu) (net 1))
 (segment (start 73.4 48) (end 75.3 46.1) (width 0.25) (layer F.Cu) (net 1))
 (segment (start 74.6 48) (end 74.7 48.1) (width 0.25) (layer F.Cu) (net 1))
 (via (at 74.7 48.1) (size 0.8) (drill 0.4) (layers F.Cu B.Cu) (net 1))
 (segment (start 71.6 48) (end 74.6 48) (width 0.25) (layer F.Cu) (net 1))
 (via (at 78.4 48.1) (size 0.8) (drill 0.4) (layers F.Cu B.Cu) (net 1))
 (segment (start 74.7 48.1) (end 78.4 48.1) (width 0.25) (layer B.Cu) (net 1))
 (segment (start 81.5 45) (end 81.5 44.7) (width 0.25) (layer F.Cu) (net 1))
 (segment (start 78.4 48.1) (end 81.5 45) (width 0.25) (layer F.Cu) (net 1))
 (segment (start 81.5 44.7) (end 88.5 44.7) (width 0.25) (layer F.Cu) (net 1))
 (segment (start 53.85 74.45) (end 53.9 74.4) (width 0.3048) (layer F.Cu) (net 13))
 (segment (start 49.5 74.45) (end 53.85 74.45) (width 0.3048) (layer F.Cu) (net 13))
 (via (at 63 57.9) (size 0.8) (drill 0.4) (layers F.Cu B.Cu) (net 13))
 (segment (start 63 55.5) (end 63 57.9) (width 0.3048) (layer F.Cu) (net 13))
 (segment (start 63 57.9) (end 61 59.9) (width 0.3048) (layer B.Cu) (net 13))
 (segment (start 61 59.9) (end 54.1 59.9) (width 0.3048) (layer B.Cu) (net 13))
 (segment (start 47.5 66.5) (end 47.5 74.4) (width 0.3048) (layer B.Cu) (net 13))
 (via (at 47.5 74.4) (size 0.8) (drill 0.4) (layers F.Cu B.Cu) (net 13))
 (segment (start 54.1 59.9) (end 47.5 66.5) (width 0.3048) (layer B.Cu) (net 13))
 (segment (start 49.45 74.4) (end 49.5 74.45) (width 0.3048) (layer F.Cu) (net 13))
 (segment (start 47.5 74.4) (end 49.45 74.4) (width 0.3048) (layer F.Cu) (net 13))
 (segment (start 65.1 79.75) (end 65.3 79.55) (width 0.3048) (layer F.Cu) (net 12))
 (segment (start 60.3 79.75) (end 65.1 79.75) (width 0.3048) (layer F.Cu) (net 12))
 (via (at 65 57.9) (size 0.8) (drill 0.4) (layers F.Cu B.Cu) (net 12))
 (segment (start 65 55.5) (end 65 57.9) (width 0.3048) (layer F.Cu) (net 12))
 (segment (start 65 57.9) (end 65 58.6) (width 0.3048) (layer B.Cu) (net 12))
 (segment (start 65 58.6) (end 62 61.6) (width 0.3048) (layer B.Cu) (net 12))
 (segment (start 62 61.6) (end 54.9 61.6) (width 0.3048) (layer B.Cu) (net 12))
 (segment (start 54.9 61.6) (end 51.2 65.3) (width 0.3048) (layer B.Cu) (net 12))
 (segment (start 51.2 65.3) (end 51.2 67.9) (width 0.3048) (layer B.Cu) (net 12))
 (via (at 60.2 77.9) (size 0.8) (drill 0.4) (layers F.Cu B.Cu) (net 12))
 (segment (start 60.2 76.9) (end 60.2 77.9) (width 0.3048) (layer B.Cu) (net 12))
 (segment (start 51.2 67.9) (end 60.2 76.9) (width 0.3048) (layer B.Cu) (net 12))
 (segment (start 60.2 79.65) (end 60.3 79.75) (width 0.3048) (layer F.Cu) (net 12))
 (segment (start 60.2 77.9) (end 60.2 79.65) (width 0.3048) (layer F.Cu) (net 12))
 (segment (start 52.45 44) (end 56.4 44) (width 0.3048) (layer F.Cu) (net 20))
 (segment (start 71.6 50) (end 74.6 50) (width 0.25) (layer F.Cu) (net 8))
 (segment (start 74.6 50) (end 77.9 46.7) (width 0.25) (layer F.Cu) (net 8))
 (segment (start 77.9 46.7) (end 77.9 42.15) (width 0.25) (layer F.Cu) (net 8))
 (segment (start 75.35 52) (end 75.4 52.05) (width 0.25) (layer F.Cu) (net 9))
 (segment (start 71.6 52) (end 75.35 52) (width 0.25) (layer F.Cu) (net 9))
 (segment (start 52.45 48) (end 56.4 48) (width 0.3048) (layer F.Cu) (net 18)))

